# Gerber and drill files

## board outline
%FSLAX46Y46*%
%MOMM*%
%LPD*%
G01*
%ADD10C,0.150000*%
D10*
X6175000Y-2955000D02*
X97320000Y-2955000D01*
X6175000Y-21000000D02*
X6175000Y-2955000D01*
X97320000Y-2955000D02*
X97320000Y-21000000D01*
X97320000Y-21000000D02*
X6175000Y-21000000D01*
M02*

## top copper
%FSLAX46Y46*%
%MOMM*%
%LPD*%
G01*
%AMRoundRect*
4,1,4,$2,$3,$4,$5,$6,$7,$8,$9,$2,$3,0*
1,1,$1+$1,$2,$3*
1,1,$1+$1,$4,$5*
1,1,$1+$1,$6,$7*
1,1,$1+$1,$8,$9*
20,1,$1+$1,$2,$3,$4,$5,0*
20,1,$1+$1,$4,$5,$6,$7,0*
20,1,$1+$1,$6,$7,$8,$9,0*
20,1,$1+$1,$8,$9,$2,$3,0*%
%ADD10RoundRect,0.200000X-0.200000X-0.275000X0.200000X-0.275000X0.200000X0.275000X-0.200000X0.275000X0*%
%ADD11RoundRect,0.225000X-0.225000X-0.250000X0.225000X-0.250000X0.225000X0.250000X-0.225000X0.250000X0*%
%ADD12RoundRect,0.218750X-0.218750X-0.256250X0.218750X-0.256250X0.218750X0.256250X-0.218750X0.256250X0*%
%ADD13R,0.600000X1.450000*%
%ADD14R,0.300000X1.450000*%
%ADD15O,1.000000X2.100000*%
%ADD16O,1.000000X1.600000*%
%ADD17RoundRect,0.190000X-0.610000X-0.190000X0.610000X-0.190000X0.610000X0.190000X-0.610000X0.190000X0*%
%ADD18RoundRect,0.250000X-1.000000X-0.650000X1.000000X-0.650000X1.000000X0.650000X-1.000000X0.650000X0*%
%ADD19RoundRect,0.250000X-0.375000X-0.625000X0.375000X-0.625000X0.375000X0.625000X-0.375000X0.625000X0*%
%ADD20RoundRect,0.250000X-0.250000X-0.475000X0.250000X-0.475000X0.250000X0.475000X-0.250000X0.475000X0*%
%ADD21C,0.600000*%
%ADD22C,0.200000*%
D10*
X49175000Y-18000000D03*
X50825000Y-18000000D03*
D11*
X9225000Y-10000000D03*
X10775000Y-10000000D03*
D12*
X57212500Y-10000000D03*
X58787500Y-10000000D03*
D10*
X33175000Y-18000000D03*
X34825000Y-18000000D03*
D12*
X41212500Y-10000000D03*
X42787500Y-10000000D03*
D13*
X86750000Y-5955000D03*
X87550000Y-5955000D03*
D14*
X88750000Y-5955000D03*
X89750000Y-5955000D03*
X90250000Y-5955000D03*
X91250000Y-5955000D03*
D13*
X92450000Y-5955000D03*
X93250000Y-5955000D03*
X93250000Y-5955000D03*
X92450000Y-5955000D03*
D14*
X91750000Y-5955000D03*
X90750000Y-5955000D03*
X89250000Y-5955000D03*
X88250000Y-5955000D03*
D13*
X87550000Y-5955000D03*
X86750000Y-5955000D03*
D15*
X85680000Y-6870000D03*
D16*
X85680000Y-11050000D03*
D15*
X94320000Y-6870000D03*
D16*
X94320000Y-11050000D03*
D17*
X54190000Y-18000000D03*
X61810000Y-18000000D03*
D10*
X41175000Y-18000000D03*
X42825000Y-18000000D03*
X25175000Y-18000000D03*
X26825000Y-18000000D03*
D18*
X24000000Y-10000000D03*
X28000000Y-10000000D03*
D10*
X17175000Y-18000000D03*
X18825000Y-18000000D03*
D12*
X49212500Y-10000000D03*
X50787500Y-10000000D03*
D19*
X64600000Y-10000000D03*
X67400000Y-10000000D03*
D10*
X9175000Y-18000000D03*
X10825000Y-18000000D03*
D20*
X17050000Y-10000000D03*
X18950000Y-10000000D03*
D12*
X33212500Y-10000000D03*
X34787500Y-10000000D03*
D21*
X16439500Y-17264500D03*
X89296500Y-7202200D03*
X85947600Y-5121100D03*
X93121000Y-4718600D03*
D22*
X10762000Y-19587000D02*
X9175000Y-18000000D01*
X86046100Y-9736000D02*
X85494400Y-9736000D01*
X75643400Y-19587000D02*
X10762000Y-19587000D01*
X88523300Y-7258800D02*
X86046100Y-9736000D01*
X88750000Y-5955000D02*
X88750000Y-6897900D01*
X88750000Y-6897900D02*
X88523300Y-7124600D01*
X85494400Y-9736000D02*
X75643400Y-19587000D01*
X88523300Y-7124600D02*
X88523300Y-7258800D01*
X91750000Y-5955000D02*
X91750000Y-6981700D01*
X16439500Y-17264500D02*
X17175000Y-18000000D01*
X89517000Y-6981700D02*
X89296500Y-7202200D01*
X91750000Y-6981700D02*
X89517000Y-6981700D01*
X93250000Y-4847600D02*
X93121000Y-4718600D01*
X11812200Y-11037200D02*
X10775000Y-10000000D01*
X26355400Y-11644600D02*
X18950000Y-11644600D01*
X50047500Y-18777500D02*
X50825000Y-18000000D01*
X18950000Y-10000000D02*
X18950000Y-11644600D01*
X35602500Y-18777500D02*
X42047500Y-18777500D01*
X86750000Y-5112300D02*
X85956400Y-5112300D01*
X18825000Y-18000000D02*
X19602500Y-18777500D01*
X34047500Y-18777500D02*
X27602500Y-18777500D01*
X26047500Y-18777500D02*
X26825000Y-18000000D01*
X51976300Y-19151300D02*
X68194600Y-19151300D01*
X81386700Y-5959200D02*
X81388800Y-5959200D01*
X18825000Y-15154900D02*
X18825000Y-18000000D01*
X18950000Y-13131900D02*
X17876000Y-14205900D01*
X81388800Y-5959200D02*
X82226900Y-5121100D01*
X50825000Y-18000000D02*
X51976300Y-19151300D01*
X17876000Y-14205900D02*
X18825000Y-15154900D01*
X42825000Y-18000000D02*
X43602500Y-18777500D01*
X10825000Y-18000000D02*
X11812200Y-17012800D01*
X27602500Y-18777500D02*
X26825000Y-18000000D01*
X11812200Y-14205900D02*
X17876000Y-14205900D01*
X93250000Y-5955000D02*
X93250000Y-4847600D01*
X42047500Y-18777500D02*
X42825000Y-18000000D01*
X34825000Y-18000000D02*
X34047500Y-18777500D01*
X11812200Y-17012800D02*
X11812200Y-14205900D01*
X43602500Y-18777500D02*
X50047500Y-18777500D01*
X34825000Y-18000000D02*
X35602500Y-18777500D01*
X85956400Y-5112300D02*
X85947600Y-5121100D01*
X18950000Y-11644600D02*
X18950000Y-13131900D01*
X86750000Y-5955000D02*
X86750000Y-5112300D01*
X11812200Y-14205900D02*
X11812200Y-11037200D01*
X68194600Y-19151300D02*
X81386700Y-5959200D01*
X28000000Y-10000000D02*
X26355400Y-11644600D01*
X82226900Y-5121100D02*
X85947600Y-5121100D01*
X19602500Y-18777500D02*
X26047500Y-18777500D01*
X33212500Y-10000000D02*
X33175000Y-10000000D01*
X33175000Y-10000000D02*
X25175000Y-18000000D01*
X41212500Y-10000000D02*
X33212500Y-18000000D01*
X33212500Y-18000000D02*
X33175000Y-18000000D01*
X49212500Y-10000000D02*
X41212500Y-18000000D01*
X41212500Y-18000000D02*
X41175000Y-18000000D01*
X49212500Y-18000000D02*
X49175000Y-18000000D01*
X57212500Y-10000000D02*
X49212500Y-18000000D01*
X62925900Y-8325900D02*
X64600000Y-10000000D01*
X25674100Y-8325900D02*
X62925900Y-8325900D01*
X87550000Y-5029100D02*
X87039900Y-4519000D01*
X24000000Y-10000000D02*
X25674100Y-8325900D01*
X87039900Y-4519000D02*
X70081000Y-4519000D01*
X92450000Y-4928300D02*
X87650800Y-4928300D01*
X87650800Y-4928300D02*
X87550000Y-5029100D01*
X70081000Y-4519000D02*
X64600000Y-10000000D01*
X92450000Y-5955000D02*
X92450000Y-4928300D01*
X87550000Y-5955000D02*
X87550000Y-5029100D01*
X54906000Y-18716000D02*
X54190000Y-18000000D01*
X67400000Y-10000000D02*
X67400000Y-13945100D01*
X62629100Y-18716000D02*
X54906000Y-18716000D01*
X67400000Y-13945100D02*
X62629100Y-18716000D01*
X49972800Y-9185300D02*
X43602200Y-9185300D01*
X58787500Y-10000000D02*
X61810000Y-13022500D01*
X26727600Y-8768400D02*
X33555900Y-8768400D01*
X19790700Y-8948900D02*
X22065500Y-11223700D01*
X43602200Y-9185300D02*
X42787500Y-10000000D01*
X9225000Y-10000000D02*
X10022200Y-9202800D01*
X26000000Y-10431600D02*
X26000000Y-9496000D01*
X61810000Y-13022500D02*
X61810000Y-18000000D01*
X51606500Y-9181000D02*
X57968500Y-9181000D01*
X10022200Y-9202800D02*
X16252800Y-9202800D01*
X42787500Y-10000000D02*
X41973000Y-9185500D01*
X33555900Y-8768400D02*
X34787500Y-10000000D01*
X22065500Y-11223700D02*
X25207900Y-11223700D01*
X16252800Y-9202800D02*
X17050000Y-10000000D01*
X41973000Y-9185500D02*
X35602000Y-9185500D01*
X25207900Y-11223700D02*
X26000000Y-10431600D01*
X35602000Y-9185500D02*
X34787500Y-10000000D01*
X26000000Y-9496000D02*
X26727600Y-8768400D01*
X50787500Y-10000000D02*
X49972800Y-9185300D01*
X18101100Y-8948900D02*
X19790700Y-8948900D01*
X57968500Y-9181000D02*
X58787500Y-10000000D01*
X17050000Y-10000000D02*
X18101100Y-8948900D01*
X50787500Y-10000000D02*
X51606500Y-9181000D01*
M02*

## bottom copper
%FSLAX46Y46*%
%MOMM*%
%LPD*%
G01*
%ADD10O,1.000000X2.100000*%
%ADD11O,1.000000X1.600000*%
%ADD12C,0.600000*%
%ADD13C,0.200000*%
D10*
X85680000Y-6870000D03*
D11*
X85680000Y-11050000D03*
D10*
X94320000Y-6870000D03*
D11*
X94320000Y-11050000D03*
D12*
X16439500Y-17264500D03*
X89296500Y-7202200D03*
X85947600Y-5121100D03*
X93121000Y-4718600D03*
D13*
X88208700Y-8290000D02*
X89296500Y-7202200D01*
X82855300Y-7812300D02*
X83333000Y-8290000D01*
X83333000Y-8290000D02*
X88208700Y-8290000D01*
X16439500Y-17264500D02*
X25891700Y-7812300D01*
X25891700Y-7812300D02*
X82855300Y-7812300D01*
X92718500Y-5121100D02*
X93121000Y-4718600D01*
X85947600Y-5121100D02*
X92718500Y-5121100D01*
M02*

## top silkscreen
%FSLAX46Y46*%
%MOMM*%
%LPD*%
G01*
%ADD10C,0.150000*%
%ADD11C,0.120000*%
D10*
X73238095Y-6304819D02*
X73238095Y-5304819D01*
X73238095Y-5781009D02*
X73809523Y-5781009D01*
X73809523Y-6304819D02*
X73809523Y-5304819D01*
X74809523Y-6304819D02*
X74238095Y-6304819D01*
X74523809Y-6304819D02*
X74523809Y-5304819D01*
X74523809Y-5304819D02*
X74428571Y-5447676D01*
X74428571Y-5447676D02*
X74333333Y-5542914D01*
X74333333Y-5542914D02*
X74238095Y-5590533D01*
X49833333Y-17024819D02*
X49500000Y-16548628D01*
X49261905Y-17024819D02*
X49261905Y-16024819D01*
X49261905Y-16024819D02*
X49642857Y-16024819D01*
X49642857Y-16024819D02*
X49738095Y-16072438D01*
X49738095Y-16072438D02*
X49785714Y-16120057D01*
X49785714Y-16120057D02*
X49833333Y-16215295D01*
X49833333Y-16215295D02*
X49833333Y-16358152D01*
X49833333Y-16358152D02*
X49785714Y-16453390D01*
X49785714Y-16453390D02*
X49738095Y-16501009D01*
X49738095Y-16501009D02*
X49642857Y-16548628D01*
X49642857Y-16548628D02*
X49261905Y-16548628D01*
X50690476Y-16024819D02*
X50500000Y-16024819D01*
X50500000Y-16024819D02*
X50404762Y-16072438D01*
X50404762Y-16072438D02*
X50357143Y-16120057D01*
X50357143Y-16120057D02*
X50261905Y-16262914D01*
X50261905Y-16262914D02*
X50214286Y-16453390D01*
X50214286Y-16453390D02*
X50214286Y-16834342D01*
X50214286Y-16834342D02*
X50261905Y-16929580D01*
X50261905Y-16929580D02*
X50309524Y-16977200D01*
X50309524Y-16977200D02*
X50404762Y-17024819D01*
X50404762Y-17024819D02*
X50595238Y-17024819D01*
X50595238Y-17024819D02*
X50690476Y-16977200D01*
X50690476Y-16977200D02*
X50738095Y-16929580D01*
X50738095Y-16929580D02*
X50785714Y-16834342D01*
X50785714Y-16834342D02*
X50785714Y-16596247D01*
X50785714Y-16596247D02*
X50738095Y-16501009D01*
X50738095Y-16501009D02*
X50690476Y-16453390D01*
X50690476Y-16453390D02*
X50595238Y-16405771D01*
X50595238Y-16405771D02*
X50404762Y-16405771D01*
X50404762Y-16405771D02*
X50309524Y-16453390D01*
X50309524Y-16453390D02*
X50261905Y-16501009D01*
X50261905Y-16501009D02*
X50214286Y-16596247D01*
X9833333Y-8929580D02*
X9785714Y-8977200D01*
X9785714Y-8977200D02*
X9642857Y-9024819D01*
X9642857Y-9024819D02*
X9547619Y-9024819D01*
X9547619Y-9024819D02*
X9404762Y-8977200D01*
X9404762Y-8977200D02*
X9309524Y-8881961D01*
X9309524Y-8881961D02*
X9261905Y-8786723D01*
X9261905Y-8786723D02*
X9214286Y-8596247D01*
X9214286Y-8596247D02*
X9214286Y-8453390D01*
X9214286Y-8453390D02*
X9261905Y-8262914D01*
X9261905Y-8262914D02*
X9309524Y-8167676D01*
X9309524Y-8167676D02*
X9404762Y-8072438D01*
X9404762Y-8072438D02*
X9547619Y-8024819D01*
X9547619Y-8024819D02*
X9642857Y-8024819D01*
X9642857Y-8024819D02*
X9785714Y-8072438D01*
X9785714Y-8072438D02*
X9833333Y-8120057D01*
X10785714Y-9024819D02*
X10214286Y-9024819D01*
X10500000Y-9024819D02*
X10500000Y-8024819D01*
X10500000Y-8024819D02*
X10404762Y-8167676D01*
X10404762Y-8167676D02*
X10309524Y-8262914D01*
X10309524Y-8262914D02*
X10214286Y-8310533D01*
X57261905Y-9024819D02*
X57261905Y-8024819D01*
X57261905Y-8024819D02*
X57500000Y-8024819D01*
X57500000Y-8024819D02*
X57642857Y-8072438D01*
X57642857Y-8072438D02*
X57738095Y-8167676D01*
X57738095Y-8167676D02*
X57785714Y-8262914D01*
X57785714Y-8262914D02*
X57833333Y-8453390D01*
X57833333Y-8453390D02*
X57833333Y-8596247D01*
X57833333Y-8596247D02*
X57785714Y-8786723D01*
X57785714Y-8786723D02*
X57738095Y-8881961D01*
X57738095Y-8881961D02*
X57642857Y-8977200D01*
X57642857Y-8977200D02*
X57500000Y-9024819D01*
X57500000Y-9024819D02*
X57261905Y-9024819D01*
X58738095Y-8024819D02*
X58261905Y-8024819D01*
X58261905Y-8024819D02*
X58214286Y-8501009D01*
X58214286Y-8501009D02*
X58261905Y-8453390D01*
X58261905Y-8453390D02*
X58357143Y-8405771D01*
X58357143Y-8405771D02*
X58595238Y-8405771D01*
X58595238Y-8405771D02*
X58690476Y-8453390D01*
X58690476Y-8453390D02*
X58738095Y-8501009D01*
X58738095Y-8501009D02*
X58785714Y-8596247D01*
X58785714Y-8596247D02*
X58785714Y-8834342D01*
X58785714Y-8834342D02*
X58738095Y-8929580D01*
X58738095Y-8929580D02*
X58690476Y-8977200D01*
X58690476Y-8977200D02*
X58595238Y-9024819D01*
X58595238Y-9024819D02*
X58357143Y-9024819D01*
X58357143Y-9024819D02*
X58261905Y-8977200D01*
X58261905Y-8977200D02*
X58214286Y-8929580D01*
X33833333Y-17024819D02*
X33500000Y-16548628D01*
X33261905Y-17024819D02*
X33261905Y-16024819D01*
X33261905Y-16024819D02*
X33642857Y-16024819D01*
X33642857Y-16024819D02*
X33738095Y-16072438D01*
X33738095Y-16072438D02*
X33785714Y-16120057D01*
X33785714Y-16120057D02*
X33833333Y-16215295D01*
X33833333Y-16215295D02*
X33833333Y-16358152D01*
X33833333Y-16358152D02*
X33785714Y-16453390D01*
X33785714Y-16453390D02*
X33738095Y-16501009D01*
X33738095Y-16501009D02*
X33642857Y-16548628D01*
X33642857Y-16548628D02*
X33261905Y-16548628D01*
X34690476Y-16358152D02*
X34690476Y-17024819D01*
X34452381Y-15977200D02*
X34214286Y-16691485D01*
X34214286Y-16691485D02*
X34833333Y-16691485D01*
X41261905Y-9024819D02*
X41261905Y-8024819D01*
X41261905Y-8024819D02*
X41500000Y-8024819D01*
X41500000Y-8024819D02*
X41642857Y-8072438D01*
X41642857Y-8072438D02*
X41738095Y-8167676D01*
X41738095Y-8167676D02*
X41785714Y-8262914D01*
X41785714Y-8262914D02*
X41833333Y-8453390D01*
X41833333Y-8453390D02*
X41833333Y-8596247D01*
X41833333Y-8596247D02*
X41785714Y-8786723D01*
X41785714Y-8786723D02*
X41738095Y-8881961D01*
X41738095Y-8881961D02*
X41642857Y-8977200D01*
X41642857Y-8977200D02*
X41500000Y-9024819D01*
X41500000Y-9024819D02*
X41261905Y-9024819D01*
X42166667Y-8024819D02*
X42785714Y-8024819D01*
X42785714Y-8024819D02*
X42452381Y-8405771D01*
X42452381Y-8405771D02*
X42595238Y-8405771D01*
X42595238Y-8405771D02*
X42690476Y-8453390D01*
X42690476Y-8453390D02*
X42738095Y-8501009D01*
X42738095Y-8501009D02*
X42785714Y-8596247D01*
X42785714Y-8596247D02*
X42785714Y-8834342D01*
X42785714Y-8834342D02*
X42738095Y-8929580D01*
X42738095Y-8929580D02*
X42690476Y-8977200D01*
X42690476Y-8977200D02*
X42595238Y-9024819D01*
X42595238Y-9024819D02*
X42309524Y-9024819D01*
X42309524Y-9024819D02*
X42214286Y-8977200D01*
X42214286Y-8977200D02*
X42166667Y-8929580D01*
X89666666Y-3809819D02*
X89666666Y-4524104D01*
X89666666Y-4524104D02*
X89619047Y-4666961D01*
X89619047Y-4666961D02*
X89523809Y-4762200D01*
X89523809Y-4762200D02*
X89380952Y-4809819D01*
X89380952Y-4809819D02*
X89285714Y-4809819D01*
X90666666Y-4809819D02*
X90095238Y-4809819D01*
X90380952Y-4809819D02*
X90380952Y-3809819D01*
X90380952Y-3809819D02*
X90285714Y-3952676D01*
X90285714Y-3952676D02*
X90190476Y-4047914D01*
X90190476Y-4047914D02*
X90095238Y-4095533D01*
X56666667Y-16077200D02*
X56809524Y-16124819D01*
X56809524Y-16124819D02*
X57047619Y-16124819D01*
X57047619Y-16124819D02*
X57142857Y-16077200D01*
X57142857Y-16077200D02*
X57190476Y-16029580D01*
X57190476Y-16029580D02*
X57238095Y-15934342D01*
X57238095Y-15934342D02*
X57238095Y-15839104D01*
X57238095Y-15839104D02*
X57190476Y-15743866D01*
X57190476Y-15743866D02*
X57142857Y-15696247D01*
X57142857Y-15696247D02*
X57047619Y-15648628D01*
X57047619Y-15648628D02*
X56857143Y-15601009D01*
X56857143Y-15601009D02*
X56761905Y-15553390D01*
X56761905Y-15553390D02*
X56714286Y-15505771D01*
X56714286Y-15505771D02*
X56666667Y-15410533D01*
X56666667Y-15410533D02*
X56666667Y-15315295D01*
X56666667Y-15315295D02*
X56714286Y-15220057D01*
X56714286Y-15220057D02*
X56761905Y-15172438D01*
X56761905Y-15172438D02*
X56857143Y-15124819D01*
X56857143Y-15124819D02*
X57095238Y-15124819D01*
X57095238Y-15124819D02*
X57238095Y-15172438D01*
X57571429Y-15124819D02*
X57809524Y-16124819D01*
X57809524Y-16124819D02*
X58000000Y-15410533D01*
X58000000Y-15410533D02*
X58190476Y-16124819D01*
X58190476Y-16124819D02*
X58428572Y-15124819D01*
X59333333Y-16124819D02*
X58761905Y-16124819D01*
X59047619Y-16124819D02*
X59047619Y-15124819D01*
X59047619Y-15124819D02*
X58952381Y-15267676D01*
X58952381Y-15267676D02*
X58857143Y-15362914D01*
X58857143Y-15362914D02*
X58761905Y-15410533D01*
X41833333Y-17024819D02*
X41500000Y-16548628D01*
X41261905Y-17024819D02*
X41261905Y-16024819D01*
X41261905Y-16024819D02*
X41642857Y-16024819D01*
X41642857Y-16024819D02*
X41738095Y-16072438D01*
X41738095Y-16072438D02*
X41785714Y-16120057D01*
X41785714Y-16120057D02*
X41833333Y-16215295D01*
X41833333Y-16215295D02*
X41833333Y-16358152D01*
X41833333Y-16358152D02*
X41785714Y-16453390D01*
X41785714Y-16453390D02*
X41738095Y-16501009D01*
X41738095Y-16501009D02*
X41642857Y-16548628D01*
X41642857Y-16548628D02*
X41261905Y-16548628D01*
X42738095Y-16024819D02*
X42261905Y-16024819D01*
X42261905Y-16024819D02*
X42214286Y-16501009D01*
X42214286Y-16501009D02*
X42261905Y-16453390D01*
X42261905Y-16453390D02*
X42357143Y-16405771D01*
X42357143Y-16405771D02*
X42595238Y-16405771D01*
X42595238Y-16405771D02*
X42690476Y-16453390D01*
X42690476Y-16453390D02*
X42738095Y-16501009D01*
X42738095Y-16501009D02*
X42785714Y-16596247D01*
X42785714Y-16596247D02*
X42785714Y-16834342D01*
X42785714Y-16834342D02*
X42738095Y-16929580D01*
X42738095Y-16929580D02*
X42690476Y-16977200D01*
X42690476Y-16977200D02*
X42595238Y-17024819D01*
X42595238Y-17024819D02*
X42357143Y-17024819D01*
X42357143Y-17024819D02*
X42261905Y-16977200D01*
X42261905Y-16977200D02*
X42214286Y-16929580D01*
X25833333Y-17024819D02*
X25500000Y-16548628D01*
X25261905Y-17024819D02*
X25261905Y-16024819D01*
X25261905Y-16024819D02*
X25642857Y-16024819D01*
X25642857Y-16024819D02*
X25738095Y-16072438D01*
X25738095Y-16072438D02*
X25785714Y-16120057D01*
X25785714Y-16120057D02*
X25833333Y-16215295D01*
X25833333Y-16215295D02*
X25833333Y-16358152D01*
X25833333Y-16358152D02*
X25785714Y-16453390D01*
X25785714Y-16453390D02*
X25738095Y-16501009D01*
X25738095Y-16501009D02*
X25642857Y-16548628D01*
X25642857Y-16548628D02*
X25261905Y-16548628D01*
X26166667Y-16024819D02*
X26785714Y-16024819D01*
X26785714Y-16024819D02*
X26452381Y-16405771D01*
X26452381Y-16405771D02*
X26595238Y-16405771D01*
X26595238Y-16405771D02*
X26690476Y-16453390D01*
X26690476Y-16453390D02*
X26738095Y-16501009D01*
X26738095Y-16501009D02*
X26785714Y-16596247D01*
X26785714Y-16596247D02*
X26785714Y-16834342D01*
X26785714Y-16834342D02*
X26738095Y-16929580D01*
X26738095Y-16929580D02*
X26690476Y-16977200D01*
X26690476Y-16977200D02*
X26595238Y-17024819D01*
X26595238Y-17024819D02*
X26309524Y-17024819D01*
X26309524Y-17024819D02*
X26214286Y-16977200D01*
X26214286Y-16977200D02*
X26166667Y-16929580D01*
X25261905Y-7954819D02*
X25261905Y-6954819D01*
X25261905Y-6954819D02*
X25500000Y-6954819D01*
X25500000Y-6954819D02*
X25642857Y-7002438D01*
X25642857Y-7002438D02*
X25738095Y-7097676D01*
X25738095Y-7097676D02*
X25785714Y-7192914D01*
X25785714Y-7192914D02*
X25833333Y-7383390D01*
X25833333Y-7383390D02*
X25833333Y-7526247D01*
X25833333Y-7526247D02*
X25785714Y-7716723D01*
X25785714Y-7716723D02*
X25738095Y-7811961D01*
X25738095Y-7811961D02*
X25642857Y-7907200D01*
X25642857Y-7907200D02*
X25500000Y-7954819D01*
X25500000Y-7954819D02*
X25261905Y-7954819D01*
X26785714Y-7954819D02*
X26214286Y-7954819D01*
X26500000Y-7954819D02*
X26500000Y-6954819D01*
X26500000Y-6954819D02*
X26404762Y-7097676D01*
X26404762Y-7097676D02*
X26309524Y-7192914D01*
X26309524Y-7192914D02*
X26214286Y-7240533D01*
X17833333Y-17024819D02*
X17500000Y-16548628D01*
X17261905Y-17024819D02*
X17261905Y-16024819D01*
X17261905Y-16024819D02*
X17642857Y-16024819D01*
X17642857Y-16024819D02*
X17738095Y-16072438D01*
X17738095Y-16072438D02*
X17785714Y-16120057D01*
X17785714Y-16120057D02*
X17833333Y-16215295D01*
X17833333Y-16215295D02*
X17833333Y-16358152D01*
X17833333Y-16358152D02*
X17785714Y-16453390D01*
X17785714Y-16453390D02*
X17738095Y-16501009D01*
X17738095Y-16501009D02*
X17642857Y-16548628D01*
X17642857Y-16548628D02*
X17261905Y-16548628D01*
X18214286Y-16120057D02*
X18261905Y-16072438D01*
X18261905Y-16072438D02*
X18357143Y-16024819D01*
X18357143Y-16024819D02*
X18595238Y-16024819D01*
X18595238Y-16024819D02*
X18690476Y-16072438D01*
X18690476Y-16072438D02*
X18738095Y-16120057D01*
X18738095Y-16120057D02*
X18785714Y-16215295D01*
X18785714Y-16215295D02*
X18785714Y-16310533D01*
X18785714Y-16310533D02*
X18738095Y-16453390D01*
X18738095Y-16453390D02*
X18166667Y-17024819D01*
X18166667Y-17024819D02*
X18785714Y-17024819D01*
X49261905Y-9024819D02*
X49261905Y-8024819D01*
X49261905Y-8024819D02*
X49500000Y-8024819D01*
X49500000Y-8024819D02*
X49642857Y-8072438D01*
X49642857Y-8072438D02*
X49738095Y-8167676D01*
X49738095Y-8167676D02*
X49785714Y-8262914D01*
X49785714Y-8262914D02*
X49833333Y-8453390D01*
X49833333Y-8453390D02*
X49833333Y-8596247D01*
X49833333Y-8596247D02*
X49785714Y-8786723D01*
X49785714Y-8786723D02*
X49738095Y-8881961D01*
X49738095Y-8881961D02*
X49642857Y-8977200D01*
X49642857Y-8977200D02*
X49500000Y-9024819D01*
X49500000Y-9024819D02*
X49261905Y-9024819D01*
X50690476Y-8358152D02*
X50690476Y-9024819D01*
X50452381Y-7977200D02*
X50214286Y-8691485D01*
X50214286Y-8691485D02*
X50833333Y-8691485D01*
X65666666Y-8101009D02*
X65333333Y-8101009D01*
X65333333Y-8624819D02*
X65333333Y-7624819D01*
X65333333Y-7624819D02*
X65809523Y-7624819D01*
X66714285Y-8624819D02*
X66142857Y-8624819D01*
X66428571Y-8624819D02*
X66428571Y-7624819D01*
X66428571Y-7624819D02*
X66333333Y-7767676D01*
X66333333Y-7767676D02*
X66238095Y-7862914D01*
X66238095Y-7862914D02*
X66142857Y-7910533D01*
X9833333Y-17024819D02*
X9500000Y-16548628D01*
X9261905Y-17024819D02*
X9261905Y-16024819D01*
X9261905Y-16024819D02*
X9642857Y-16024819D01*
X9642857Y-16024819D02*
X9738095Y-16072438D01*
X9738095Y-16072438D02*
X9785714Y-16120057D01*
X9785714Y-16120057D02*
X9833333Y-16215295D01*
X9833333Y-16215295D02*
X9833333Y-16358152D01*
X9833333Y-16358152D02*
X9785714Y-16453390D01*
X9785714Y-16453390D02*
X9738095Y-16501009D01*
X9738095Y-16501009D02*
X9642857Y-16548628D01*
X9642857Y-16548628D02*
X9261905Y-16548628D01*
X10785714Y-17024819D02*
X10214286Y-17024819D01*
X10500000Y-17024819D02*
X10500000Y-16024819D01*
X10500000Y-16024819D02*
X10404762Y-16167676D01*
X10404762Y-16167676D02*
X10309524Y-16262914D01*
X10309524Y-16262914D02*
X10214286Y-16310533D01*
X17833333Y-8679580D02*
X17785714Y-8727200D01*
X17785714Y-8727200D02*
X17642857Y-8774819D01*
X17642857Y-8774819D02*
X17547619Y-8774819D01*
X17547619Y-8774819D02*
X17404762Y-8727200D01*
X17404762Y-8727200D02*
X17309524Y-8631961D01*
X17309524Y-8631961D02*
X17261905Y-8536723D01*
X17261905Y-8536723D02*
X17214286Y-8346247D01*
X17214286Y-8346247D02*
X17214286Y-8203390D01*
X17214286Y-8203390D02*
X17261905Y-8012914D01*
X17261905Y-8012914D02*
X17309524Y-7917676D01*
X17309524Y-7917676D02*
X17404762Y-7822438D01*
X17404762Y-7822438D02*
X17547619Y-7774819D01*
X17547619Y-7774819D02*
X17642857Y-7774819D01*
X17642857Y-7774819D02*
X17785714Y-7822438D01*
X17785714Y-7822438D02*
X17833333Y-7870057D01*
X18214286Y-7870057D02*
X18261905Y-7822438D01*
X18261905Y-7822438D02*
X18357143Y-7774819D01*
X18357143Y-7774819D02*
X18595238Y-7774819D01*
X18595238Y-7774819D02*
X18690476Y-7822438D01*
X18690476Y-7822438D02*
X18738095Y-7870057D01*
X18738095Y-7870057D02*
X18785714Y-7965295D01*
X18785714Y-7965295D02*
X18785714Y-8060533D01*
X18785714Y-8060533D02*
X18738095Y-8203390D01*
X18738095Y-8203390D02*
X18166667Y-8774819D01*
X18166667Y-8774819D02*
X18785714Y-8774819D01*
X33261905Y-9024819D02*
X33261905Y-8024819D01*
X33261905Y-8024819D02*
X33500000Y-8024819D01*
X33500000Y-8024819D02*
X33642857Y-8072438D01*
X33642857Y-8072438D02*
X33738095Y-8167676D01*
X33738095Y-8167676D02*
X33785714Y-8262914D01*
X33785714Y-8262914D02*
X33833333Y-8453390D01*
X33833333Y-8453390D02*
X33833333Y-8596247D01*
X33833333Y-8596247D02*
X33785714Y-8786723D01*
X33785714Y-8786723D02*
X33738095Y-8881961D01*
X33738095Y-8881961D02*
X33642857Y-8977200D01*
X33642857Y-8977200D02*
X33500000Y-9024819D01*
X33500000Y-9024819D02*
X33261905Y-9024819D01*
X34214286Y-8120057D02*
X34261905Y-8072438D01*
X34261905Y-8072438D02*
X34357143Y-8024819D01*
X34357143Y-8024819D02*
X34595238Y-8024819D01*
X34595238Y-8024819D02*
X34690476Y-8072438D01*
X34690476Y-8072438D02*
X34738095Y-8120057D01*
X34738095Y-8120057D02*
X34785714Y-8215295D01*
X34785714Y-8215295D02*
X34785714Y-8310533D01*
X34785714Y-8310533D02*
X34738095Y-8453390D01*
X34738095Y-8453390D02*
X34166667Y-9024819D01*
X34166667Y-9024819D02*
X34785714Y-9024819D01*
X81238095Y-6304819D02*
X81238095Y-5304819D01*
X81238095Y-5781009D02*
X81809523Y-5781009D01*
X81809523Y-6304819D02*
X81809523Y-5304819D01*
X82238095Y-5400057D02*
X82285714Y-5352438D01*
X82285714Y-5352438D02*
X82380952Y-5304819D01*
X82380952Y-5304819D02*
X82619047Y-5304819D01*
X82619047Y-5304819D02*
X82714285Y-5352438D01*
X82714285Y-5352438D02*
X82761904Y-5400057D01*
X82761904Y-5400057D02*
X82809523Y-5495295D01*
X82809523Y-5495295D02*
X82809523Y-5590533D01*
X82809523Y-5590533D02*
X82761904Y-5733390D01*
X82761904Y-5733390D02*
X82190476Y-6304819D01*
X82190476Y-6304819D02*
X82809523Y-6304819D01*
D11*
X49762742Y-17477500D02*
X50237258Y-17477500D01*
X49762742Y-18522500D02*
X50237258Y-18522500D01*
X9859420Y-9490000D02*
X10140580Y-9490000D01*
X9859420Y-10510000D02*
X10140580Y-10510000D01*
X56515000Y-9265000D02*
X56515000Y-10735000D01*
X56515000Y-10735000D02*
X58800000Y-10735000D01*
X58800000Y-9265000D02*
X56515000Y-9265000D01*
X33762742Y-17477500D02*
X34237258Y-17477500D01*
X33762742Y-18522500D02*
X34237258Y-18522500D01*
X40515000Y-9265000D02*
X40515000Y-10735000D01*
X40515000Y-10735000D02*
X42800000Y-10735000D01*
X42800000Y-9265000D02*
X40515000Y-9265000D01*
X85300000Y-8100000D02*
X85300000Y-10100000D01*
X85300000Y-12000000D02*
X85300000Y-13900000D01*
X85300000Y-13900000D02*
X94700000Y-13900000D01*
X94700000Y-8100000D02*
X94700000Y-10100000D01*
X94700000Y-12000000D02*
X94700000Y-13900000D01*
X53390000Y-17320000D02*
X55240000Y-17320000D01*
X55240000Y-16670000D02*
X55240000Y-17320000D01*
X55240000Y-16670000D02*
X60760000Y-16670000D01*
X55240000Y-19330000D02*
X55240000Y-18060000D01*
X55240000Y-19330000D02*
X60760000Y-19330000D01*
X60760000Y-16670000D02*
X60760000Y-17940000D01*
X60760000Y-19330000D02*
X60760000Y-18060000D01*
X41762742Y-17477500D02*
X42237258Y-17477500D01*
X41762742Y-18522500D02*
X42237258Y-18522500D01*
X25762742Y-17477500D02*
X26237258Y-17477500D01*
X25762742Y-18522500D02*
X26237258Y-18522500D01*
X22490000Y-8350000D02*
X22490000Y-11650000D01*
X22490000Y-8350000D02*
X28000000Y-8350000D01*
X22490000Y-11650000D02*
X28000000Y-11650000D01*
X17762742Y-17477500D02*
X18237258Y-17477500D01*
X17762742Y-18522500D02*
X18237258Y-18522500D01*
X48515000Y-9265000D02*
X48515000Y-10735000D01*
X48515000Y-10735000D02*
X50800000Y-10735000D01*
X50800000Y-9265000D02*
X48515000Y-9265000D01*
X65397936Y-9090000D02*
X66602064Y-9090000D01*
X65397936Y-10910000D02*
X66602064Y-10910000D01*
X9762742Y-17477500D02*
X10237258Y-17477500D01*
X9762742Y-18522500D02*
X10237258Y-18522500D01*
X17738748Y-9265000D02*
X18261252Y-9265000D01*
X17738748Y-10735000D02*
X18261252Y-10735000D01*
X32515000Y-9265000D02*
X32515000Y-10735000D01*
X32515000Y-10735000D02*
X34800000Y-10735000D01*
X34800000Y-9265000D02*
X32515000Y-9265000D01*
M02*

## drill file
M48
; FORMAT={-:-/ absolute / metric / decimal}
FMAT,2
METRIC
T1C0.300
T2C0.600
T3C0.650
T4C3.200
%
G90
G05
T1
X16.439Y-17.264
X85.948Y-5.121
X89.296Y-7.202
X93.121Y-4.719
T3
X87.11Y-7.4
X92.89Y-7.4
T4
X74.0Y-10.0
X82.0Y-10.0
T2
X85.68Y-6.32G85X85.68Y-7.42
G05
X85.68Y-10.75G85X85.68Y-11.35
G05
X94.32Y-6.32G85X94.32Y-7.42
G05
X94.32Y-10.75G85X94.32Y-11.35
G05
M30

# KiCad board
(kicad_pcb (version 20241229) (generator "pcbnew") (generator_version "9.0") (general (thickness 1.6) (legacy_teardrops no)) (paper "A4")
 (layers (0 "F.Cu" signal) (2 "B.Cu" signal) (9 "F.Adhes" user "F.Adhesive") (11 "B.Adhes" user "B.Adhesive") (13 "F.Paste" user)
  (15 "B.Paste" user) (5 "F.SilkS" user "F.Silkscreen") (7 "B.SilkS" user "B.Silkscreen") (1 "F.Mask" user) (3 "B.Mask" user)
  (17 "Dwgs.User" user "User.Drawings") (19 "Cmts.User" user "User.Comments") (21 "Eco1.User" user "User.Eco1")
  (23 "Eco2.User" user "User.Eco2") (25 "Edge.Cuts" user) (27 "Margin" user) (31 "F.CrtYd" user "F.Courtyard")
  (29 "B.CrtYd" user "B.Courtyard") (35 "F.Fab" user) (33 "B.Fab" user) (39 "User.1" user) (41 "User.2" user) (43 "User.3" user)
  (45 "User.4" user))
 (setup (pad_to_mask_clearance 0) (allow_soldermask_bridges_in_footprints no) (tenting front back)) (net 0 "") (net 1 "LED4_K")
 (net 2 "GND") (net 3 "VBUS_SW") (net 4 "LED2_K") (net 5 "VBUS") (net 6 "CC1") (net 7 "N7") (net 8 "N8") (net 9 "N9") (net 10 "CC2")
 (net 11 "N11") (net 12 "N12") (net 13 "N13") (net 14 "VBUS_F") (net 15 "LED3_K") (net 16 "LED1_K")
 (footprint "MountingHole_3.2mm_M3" (layer "F.Cu") (at 74 10)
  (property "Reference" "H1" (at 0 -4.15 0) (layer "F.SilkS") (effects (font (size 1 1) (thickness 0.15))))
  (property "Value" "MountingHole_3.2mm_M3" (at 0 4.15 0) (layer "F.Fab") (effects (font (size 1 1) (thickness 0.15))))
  (pad "" np_thru_hole circle (at 0 0) (size 3.2 3.2) (drill 3.2) (layers "*.Cu" "*.Mask")))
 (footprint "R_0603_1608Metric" (layer "F.Cu") (at 50 18)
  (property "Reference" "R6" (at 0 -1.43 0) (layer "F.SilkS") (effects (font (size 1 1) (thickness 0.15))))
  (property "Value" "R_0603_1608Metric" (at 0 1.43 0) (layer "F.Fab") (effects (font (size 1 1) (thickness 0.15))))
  (fp_line (start -0.237258 -0.5225) (end 0.237258 -0.5225) (stroke (width 0.12) (type solid)) (layer "F.SilkS"))
  (fp_line (start -0.237258 0.5225) (end 0.237258 0.5225) (stroke (width 0.12) (type solid)) (layer "F.SilkS"))
  (pad "1" smd roundrect (at -0.825 0) (size 0.8 0.95) (layers "F.Cu" "F.Mask" "F.Paste") (roundrect_rratio 0.25) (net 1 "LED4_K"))
  (pad "2" smd roundrect (at 0.825 0) (size 0.8 0.95) (layers "F.Cu" "F.Mask" "F.Paste") (roundrect_rratio 0.25) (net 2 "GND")))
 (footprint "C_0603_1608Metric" (layer "F.Cu") (at 10 10)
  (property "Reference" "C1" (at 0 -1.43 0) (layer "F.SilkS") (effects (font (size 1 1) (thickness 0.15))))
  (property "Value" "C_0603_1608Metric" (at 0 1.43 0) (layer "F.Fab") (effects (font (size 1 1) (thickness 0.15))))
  (fp_line (start -0.14058 -0.51) (end 0.14058 -0.51) (stroke (width 0.12) (type solid)) (layer "F.SilkS"))
  (fp_line (start -0.14058 0.51) (end 0.14058 0.51) (stroke (width 0.12) (type solid)) (layer "F.SilkS"))
  (pad "1" smd roundrect (at -0.775 0) (size 0.9 0.95) (layers "F.Cu" "F.Mask" "F.Paste") (roundrect_rratio 0.25) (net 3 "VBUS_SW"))
  (pad "2" smd roundrect (at 0.775 0) (size 0.9 0.95) (layers "F.Cu" "F.Mask" "F.Paste") (roundrect_rratio 0.25) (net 2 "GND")))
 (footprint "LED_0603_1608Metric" (layer "F.Cu") (at 58 10)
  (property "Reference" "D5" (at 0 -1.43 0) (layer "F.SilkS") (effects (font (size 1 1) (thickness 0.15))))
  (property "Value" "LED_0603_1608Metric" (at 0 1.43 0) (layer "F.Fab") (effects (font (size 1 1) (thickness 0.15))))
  (fp_line (start -1.485 -0.735) (end -1.485 0.735) (stroke (width 0.12) (type solid)) (layer "F.SilkS"))
  (fp_line (start -1.485 0.735) (end 0.8 0.735) (stroke (width 0.12) (type solid)) (layer "F.SilkS"))
  (fp_line (start 0.8 -0.735) (end -1.485 -0.735) (stroke (width 0.12) (type solid)) (layer "F.SilkS"))
  (pad "1" smd roundrect (at -0.7875 0) (size 0.875 0.95) (layers "F.Cu" "F.Mask" "F.Paste") (roundrect_rratio 0.25) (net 1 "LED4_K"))
  (pad "2" smd roundrect (at 0.7875 0) (size 0.875 0.95) (layers "F.Cu" "F.Mask" "F.Paste") (roundrect_rratio 0.25) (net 3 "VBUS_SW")))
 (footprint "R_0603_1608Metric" (layer "F.Cu") (at 34 18)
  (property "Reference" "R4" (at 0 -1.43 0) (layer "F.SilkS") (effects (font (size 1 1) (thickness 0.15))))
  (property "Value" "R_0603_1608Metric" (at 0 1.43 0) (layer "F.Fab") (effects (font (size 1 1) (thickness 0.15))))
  (fp_line (start -0.237258 -0.5225) (end 0.237258 -0.5225) (stroke (width 0.12) (type solid)) (layer "F.SilkS"))
  (fp_line (start -0.237258 0.5225) (end 0.237258 0.5225) (stroke (width 0.12) (type solid)) (layer "F.SilkS"))
  (pad "1" smd roundrect (at -0.825 0) (size 0.8 0.95) (layers "F.Cu" "F.Mask" "F.Paste") (roundrect_rratio 0.25) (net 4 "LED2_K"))
  (pad "2" smd roundrect (at 0.825 0) (size 0.8 0.95) (layers "F.Cu" "F.Mask" "F.Paste") (roundrect_rratio 0.25) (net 2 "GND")))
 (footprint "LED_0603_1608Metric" (layer "F.Cu") (at 42 10)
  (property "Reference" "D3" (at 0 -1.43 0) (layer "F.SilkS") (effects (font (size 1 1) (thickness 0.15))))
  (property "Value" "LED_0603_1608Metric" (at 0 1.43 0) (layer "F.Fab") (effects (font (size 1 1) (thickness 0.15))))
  (fp_line (start -1.485 -0.735) (end -1.485 0.735) (stroke (width 0.12) (type solid)) (layer "F.SilkS"))
  (fp_line (start -1.485 0.735) (end 0.8 0.735) (stroke (width 0.12) (type solid)) (layer "F.SilkS"))
  (fp_line (start 0.8 -0.735) (end -1.485 -0.735) (stroke (width 0.12) (type solid)) (layer "F.SilkS"))
  (pad "1" smd roundrect (at -0.7875 0) (size 0.875 0.95) (layers "F.Cu" "F.Mask" "F.Paste") (roundrect_rratio 0.25) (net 4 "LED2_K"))
  (pad "2" smd roundrect (at 0.7875 0) (size 0.875 0.95) (layers "F.Cu" "F.Mask" "F.Paste") (roundrect_rratio 0.25) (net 3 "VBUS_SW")))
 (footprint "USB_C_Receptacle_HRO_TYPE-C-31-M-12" (layer "F.Cu") (at 90 10)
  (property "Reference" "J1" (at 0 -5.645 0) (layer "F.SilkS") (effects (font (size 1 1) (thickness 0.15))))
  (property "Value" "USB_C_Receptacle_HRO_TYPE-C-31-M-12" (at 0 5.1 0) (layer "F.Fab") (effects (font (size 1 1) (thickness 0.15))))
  (fp_line (start -4.7 -1.9) (end -4.7 0.1) (stroke (width 0.12) (type solid)) (layer "F.SilkS"))
  (fp_line (start -4.7 2) (end -4.7 3.9) (stroke (width 0.12) (type solid)) (layer "F.SilkS"))
  (fp_line (start -4.7 3.9) (end 4.7 3.9) (stroke (width 0.12) (type solid)) (layer "F.SilkS"))
  (fp_line (start 4.7 -1.9) (end 4.7 0.1) (stroke (width 0.12) (type solid)) (layer "F.SilkS"))
  (fp_line (start 4.7 2) (end 4.7 3.9) (stroke (width 0.12) (type solid)) (layer "F.SilkS"))
  (pad "" np_thru_hole circle (at -2.89 -2.6) (size 0.65 0.65) (drill 0.65) (layers "*.Cu" "*.Mask"))
  (pad "" np_thru_hole circle (at 2.89 -2.6) (size 0.65 0.65) (drill 0.65) (layers "*.Cu" "*.Mask"))
  (pad "A1" smd rect (at -3.25 -4.045) (size 0.6 1.45) (layers "F.Cu" "F.Mask" "F.Paste") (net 2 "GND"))
  (pad "A4" smd rect (at -2.45 -4.045) (size 0.6 1.45) (layers "F.Cu" "F.Mask" "F.Paste") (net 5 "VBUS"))
  (pad "A5" smd rect (at -1.25 -4.045) (size 0.3 1.45) (layers "F.Cu" "F.Mask" "F.Paste") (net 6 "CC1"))
  (pad "A6" smd rect (at -0.25 -4.045) (size 0.3 1.45) (layers "F.Cu" "F.Mask" "F.Paste") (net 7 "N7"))
  (pad "A7" smd rect (at 0.25 -4.045) (size 0.3 1.45) (layers "F.Cu" "F.Mask" "F.Paste") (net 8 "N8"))
  (pad "A8" smd rect (at 1.25 -4.045) (size 0.3 1.45) (layers "F.Cu" "F.Mask" "F.Paste") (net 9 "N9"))
  (pad "A9" smd rect (at 2.45 -4.045) (size 0.6 1.45) (layers "F.Cu" "F.Mask" "F.Paste") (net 5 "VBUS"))
  (pad "A12" smd rect (at 3.25 -4.045) (size 0.6 1.45) (layers "F.Cu" "F.Mask" "F.Paste") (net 2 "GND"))
  (pad "B1" smd rect (at 3.25 -4.045) (size 0.6 1.45) (layers "F.Cu" "F.Mask" "F.Paste") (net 2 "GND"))
  (pad "B4" smd rect (at 2.45 -4.045) (size 0.6 1.45) (layers "F.Cu" "F.Mask" "F.Paste") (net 5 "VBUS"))
  (pad "B5" smd rect (at 1.75 -4.045) (size 0.3 1.45) (layers "F.Cu" "F.Mask" "F.Paste") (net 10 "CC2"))
  (pad "B6" smd rect (at 0.75 -4.045) (size 0.3 1.45) (layers "F.Cu" "F.Mask" "F.Paste") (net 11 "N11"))
  (pad "B7" smd rect (at -0.75 -4.045) (size 0.3 1.45) (layers "F.Cu" "F.Mask" "F.Paste") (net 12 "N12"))
  (pad "B8" smd rect (at -1.75 -4.045) (size 0.3 1.45) (layers "F.Cu" "F.Mask" "F.Paste") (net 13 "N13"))
  (pad "B9" smd rect (at -2.45 -4.045) (size 0.6 1.45) (layers "F.Cu" "F.Mask" "F.Paste") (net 5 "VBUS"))
  (pad "B12" smd rect (at -3.25 -4.045) (size 0.6 1.45) (layers "F.Cu" "F.Mask" "F.Paste") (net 2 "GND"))
  (pad "S1" thru_hole oval (at -4.32 -3.13) (size 1 2.1) (drill oval 0.6 1.7) (layers "*.Cu" "*.Mask") (remove_unused_layers no))
  (pad "S1" thru_hole oval (at -4.32 1.05) (size 1 1.6) (drill oval 0.6 1.2) (layers "*.Cu" "*.Mask") (remove_unused_layers no))
  (pad "S1" thru_hole oval (at 4.32 -3.13) (size 1 2.1) (drill oval 0.6 1.7) (layers "*.Cu" "*.Mask") (remove_unused_layers no))
  (pad "S1" thru_hole oval (at 4.32 1.05) (size 1 1.6) (drill oval 0.6 1.2) (layers "*.Cu" "*.Mask") (remove_unused_layers no)))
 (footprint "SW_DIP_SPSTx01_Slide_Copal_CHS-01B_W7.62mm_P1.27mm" (layer "F.Cu") (at 58 18)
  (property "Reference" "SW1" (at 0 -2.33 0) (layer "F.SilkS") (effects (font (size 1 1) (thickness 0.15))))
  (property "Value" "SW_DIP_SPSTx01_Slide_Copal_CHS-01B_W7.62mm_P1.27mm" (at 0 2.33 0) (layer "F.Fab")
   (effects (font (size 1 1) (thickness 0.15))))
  (fp_line (start -4.61 -0.68) (end -2.76 -0.68) (stroke (width 0.12) (type solid)) (layer "F.SilkS"))
  (fp_line (start -2.76 -1.33) (end -2.76 -0.68) (stroke (width 0.12) (type solid)) (layer "F.SilkS"))
  (fp_line (start -2.76 -1.33) (end 2.76 -1.33) (stroke (width 0.12) (type solid)) (layer "F.SilkS"))
  (fp_line (start -2.76 1.33) (end -2.76 0.06) (stroke (width 0.12) (type solid)) (layer "F.SilkS"))
  (fp_line (start -2.76 1.33) (end 2.76 1.33) (stroke (width 0.12) (type solid)) (layer "F.SilkS"))
  (fp_line (start 2.76 -1.33) (end 2.76 -0.06) (stroke (width 0.12) (type solid)) (layer "F.SilkS"))
  (fp_line (start 2.76 1.33) (end 2.76 0.06) (stroke (width 0.12) (type solid)) (layer "F.SilkS"))
  (pad "1" smd roundrect (at -3.81 0) (size 1.6 0.76) (layers "F.Cu" "F.Mask" "F.Paste") (roundrect_rratio 0.25) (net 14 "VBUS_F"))
  (pad "2" smd roundrect (at 3.81 0) (size 1.6 0.76) (layers "F.Cu" "F.Mask" "F.Paste") (roundrect_rratio 0.25) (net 3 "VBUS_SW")))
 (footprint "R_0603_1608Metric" (layer "F.Cu") (at 42 18)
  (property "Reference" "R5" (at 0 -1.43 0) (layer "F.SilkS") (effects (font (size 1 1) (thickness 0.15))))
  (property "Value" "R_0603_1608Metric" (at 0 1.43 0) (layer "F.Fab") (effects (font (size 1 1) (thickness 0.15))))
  (fp_line (start -0.237258 -0.5225) (end 0.237258 -0.5225) (stroke (width 0.12) (type solid)) (layer "F.SilkS"))
  (fp_line (start -0.237258 0.5225) (end 0.237258 0.5225) (stroke (width 0.12) (type solid)) (layer "F.SilkS"))
  (pad "1" smd roundrect (at -0.825 0) (size 0.8 0.95) (layers "F.Cu" "F.Mask" "F.Paste") (roundrect_rratio 0.25) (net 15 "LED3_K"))
  (pad "2" smd roundrect (at 0.825 0) (size 0.8 0.95) (layers "F.Cu" "F.Mask" "F.Paste") (roundrect_rratio 0.25) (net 2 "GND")))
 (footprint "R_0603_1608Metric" (layer "F.Cu") (at 26 18)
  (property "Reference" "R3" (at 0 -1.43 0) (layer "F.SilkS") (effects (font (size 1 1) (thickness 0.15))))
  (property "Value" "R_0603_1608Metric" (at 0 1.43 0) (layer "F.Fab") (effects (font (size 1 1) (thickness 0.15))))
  (fp_line (start -0.237258 -0.5225) (end 0.237258 -0.5225) (stroke (width 0.12) (type solid)) (layer "F.SilkS"))
  (fp_line (start -0.237258 0.5225) (end 0.237258 0.5225) (stroke (width 0.12) (type solid)) (layer "F.SilkS"))
  (pad "1" smd roundrect (at -0.825 0) (size 0.8 0.95) (layers "F.Cu" "F.Mask" "F.Paste") (roundrect_rratio 0.25) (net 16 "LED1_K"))
  (pad "2" smd roundrect (at 0.825 0) (size 0.8 0.95) (layers "F.Cu" "F.Mask" "F.Paste") (roundrect_rratio 0.25) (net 2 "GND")))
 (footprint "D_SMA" (layer "F.Cu") (at 26 10)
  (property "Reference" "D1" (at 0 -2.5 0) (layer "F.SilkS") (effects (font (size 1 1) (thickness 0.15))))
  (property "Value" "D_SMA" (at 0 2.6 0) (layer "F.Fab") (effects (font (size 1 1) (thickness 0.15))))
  (fp_line (start -3.51 -1.65) (end -3.51 1.65) (stroke (width 0.12) (type solid)) (layer "F.SilkS"))
  (fp_line (start -3.51 -1.65) (end 2 -1.65) (stroke (width 0.12) (type solid)) (layer "F.SilkS"))
  (fp_line (start -3.51 1.65) (end 2 1.65) (stroke (width 0.12) (type solid)) (layer "F.SilkS"))
  (pad "1" smd roundrect (at -2 0) (size 2.5 1.8) (layers "F.Cu" "F.Mask" "F.Paste") (roundrect_rratio 0.1388888889) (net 5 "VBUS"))
  (pad "2" smd roundrect (at 2 0) (size 2.5 1.8) (layers "F.Cu" "F.Mask" "F.Paste") (roundrect_rratio 0.1388888889) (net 2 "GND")))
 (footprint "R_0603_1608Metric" (layer "F.Cu") (at 18 18)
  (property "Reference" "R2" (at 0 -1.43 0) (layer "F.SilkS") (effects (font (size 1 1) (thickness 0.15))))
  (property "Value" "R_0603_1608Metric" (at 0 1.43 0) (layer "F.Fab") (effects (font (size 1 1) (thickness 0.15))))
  (fp_line (start -0.237258 -0.5225) (end 0.237258 -0.5225) (stroke (width 0.12) (type solid)) (layer "F.SilkS"))
  (fp_line (start -0.237258 0.5225) (end 0.237258 0.5225) (stroke (width 0.12) (type solid)) (layer "F.SilkS"))
  (pad "1" smd roundrect (at -0.825 0) (size 0.8 0.95) (layers "F.Cu" "F.Mask" "F.Paste") (roundrect_rratio 0.25) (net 10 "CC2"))
  (pad "2" smd roundrect (at 0.825 0) (size 0.8 0.95) (layers "F.Cu" "F.Mask" "F.Paste") (roundrect_rratio 0.25) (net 2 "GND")))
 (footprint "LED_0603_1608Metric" (layer "F.Cu") (at 50 10)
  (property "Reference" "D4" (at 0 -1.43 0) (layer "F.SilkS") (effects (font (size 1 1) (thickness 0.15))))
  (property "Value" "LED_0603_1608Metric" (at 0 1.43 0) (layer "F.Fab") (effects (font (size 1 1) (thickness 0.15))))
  (fp_line (start -1.485 -0.735) (end -1.485 0.735) (stroke (width 0.12) (type solid)) (layer "F.SilkS"))
  (fp_line (start -1.485 0.735) (end 0.8 0.735) (stroke (width 0.12) (type solid)) (layer "F.SilkS"))
  (fp_line (start 0.8 -0.735) (end -1.485 -0.735) (stroke (width 0.12) (type solid)) (layer "F.SilkS"))
  (pad "1" smd roundrect (at -0.7875 0) (size 0.875 0.95) (layers "F.Cu" "F.Mask" "F.Paste") (roundrect_rratio 0.25) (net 15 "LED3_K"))
  (pad "2" smd roundrect (at 0.7875 0) (size 0.875 0.95) (layers "F.Cu" "F.Mask" "F.Paste") (roundrect_rratio 0.25) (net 3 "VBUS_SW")))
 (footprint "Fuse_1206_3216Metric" (layer "F.Cu") (at 66 10)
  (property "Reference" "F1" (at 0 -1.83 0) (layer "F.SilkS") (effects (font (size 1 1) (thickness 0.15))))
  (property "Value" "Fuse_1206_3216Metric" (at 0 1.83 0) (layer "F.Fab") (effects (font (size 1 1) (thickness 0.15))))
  (fp_line (start -0.602064 -0.91) (end 0.602064 -0.91) (stroke (width 0.12) (type solid)) (layer "F.SilkS"))
  (fp_line (start -0.602064 0.91) (end 0.602064 0.91) (stroke (width 0.12) (type solid)) (layer "F.SilkS"))
  (pad "1" smd roundrect (at -1.4 0) (size 1.25 1.75) (layers "F.Cu" "F.Mask" "F.Paste") (roundrect_rratio 0.2) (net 5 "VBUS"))
  (pad "2" smd roundrect (at 1.4 0) (size 1.25 1.75) (layers "F.Cu" "F.Mask" "F.Paste") (roundrect_rratio 0.2) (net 14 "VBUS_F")))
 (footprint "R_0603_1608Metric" (layer "F.Cu") (at 10 18)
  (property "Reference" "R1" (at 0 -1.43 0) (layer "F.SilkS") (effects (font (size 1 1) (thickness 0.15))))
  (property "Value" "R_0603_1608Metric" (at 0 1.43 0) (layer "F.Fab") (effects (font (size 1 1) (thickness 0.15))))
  (fp_line (start -0.237258 -0.5225) (end 0.237258 -0.5225) (stroke (width 0.12) (type solid)) (layer "F.SilkS"))
  (fp_line (start -0.237258 0.5225) (end 0.237258 0.5225) (stroke (width 0.12) (type solid)) (layer "F.SilkS"))
  (pad "1" smd roundrect (at -0.825 0) (size 0.8 0.95) (layers "F.Cu" "F.Mask" "F.Paste") (roundrect_rratio 0.25) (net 6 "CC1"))
  (pad "2" smd roundrect (at 0.825 0) (size 0.8 0.95) (layers "F.Cu" "F.Mask" "F.Paste") (roundrect_rratio 0.25) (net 2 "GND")))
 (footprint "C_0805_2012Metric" (layer "F.Cu") (at 18 10)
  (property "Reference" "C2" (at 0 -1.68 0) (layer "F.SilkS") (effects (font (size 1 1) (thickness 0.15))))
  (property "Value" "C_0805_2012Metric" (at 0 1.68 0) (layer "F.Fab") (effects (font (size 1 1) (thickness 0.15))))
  (fp_line (start -0.261252 -0.735) (end 0.261252 -0.735) (stroke (width 0.12) (type solid)) (layer "F.SilkS"))
  (fp_line (start -0.261252 0.735) (end 0.261252 0.735) (stroke (width 0.12) (type solid)) (layer "F.SilkS"))
  (pad "1" smd roundrect (at -0.95 0) (size 1 1.45) (layers "F.Cu" "F.Mask" "F.Paste") (roundrect_rratio 0.25) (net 3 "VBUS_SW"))
  (pad "2" smd roundrect (at 0.95 0) (size 1 1.45) (layers "F.Cu" "F.Mask" "F.Paste") (roundrect_rratio 0.25) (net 2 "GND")))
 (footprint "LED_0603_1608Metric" (layer "F.Cu") (at 34 10)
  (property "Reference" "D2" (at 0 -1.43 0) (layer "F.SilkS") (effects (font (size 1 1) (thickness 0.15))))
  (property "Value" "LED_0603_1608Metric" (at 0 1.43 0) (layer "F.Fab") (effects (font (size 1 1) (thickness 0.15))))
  (fp_line (start -1.485 -0.735) (end -1.485 0.735) (stroke (width 0.12) (type solid)) (layer "F.SilkS"))
  (fp_line (start -1.485 0.735) (end 0.8 0.735) (stroke (width 0.12) (type solid)) (layer "F.SilkS"))
  (fp_line (start 0.8 -0.735) (end -1.485 -0.735) (stroke (width 0.12) (type solid)) (layer "F.SilkS"))
  (pad "1" smd roundrect (at -0.7875 0) (size 0.875 0.95) (layers "F.Cu" "F.Mask" "F.Paste") (roundrect_rratio 0.25) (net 16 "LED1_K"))
  (pad "2" smd roundrect (at 0.7875 0) (size 0.875 0.95) (layers "F.Cu" "F.Mask" "F.Paste") (roundrect_rratio 0.25) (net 3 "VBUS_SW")))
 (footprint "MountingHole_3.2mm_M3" (layer "F.Cu") (at 82 10)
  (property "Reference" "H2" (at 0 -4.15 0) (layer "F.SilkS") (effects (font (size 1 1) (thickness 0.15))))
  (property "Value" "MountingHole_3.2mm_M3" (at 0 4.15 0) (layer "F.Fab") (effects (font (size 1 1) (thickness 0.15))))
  (pad "" np_thru_hole circle (at 0 0) (size 3.2 3.2) (drill 3.2) (layers "*.Cu" "*.Mask")))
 (gr_line (start 6.175 2.955) (end 97.32 2.955) (stroke (width 0.15) (type default)) (layer "Edge.Cuts"))
 (gr_line (start 6.175 21) (end 6.175 2.955) (stroke (width 0.15) (type default)) (layer "Edge.Cuts"))
 (gr_line (start 97.32 2.955) (end 97.32 21) (stroke (width 0.15) (type default)) (layer "Edge.Cuts"))
 (gr_line (start 97.32 21) (end 6.175 21) (stroke (width 0.15) (type default)) (layer "Edge.Cuts"))
 (segment (start 10.762 19.587) (end 9.175 18) (width 0.2) (layer "F.Cu") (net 6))
 (segment (start 86.0461 9.736) (end 85.4944 9.736) (width 0.2) (layer "F.Cu") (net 6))
 (segment (start 75.6434 19.587) (end 10.762 19.587) (width 0.2) (layer "F.Cu") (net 6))
 (segment (start 88.5233 7.2588) (end 86.0461 9.736) (width 0.2) (layer "F.Cu") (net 6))
 (segment (start 88.75 5.955) (end 88.75 6.8979) (width 0.2) (layer "F.Cu") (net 6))
 (segment (start 88.75 6.8979) (end 88.5233 7.1246) (width 0.2) (layer "F.Cu") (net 6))
 (segment (start 85.4944 9.736) (end 75.6434 19.587) (width 0.2) (layer "F.Cu") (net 6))
 (segment (start 88.5233 7.1246) (end 88.5233 7.2588) (width 0.2) (layer "F.Cu") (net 6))
 (segment (start 91.75 5.955) (end 91.75 6.9817) (width 0.2) (layer "F.Cu") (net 10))
 (segment (start 16.4395 17.2645) (end 17.175 18) (width 0.2) (layer "F.Cu") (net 10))
 (segment (start 89.517 6.9817) (end 89.2965 7.2022) (width 0.2) (layer "F.Cu") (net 10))
 (segment (start 91.75 6.9817) (end 89.517 6.9817) (width 0.2) (layer "F.Cu") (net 10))
 (via (at 16.4395 17.2645) (size 0.6) (drill 0.3) (layers "F.Cu" "B.Cu") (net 10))
 (via (at 89.2965 7.2022) (size 0.6) (drill 0.3) (layers "F.Cu" "B.Cu") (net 10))
 (segment (start 88.2087 8.29) (end 89.2965 7.2022) (width 0.2) (layer "B.Cu") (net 10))
 (segment (start 82.8553 7.8123) (end 83.333 8.29) (width 0.2) (layer "B.Cu") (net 10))
 (segment (start 83.333 8.29) (end 88.2087 8.29) (width 0.2) (layer "B.Cu") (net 10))
 (segment (start 16.4395 17.2645) (end 25.8917 7.8123) (width 0.2) (layer "B.Cu") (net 10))
 (segment (start 25.8917 7.8123) (end 82.8553 7.8123) (width 0.2) (layer "B.Cu") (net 10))
 (segment (start 93.25 4.8476) (end 93.121 4.7186) (width 0.2) (layer "F.Cu") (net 2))
 (segment (start 11.8122 11.0372) (end 10.775 10) (width 0.2) (layer "F.Cu") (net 2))
 (segment (start 26.3554 11.6446) (end 18.95 11.6446) (width 0.2) (layer "F.Cu") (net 2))
 (segment (start 50.0475 18.7775) (end 50.825 18) (width 0.2) (layer "F.Cu") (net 2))
 (segment (start 18.95 10) (end 18.95 11.6446) (width 0.2) (layer "F.Cu") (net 2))
 (segment (start 35.6025 18.7775) (end 42.0475 18.7775) (width 0.2) (layer "F.Cu") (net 2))
 (segment (start 86.75 5.1123) (end 85.9564 5.1123) (width 0.2) (layer "F.Cu") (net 2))
 (segment (start 18.825 18) (end 19.6025 18.7775) (width 0.2) (layer "F.Cu") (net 2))
 (segment (start 34.0475 18.7775) (end 27.6025 18.7775) (width 0.2) (layer "F.Cu") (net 2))
 (segment (start 26.0475 18.7775) (end 26.825 18) (width 0.2) (layer "F.Cu") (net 2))
 (segment (start 51.9763 19.1513) (end 68.1946 19.1513) (width 0.2) (layer "F.Cu") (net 2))
 (segment (start 81.3867 5.9592) (end 81.3888 5.9592) (width 0.2) (layer "F.Cu") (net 2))
 (segment (start 18.825 15.1549) (end 18.825 18) (width 0.2) (layer "F.Cu") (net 2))
 (segment (start 18.95 13.1319) (end 17.876 14.2059) (width 0.2) (layer "F.Cu") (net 2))
 (segment (start 81.3888 5.9592) (end 82.2269 5.1211) (width 0.2) (layer "F.Cu") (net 2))
 (segment (start 50.825 18) (end 51.9763 19.1513) (width 0.2) (layer "F.Cu") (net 2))
 (segment (start 17.876 14.2059) (end 18.825 15.1549) (width 0.2) (layer "F.Cu") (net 2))
 (segment (start 42.825 18) (end 43.6025 18.7775) (width 0.2) (layer "F.Cu") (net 2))
 (segment (start 10.825 18) (end 11.8122 17.0128) (width 0.2) (layer "F.Cu") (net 2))
 (segment (start 27.6025 18.7775) (end 26.825 18) (width 0.2) (layer "F.Cu") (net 2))
 (segment (start 11.8122 14.2059) (end 17.876 14.2059) (width 0.2) (layer "F.Cu") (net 2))
 (segment (start 93.25 5.955) (end 93.25 4.8476) (width 0.2) (layer "F.Cu") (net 2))
 (segment (start 42.0475 18.7775) (end 42.825 18) (width 0.2) (layer "F.Cu") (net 2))
 (segment (start 34.825 18) (end 34.0475 18.7775) (width 0.2) (layer "F.Cu") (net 2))
 (segment (start 11.8122 17.0128) (end 11.8122 14.2059) (width 0.2) (layer "F.Cu") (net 2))
 (segment (start 43.6025 18.7775) (end 50.0475 18.7775) (width 0.2) (layer "F.Cu") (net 2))
 (segment (start 34.825 18) (end 35.6025 18.7775) (width 0.2) (layer "F.Cu") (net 2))
 (segment (start 85.9564 5.1123) (end 85.9476 5.1211) (width 0.2) (layer "F.Cu") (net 2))
 (segment (start 18.95 11.6446) (end 18.95 13.1319) (width 0.2) (layer "F.Cu") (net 2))
 (segment (start 86.75 5.955) (end 86.75 5.1123) (width 0.2) (layer "F.Cu") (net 2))
 (segment (start 11.8122 14.2059) (end 11.8122 11.0372) (width 0.2) (layer "F.Cu") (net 2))
 (segment (start 68.1946 19.1513) (end 81.3867 5.9592) (width 0.2) (layer "F.Cu") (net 2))
 (segment (start 28 10) (end 26.3554 11.6446) (width 0.2) (layer "F.Cu") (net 2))
 (segment (start 82.2269 5.1211) (end 85.9476 5.1211) (width 0.2) (layer "F.Cu") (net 2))
 (segment (start 19.6025 18.7775) (end 26.0475 18.7775) (width 0.2) (layer "F.Cu") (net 2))
 (via (at 85.9476 5.1211) (size 0.6) (drill 0.3) (layers "F.Cu" "B.Cu") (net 2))
 (via (at 93.121 4.7186) (size 0.6) (drill 0.3) (layers "F.Cu" "B.Cu") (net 2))
 (segment (start 92.7185 5.1211) (end 93.121 4.7186) (width 0.2) (layer "B.Cu") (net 2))
 (segment (start 85.9476 5.1211) (end 92.7185 5.1211) (width 0.2) (layer "B.Cu") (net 2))
 (segment (start 33.2125 10) (end 33.175 10) (width 0.2) (layer "F.Cu") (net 16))
 (segment (start 33.175 10) (end 25.175 18) (width 0.2) (layer "F.Cu") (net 16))
 (segment (start 41.2125 10) (end 33.2125 18) (width 0.2) (layer "F.Cu") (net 4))
 (segment (start 33.2125 18) (end 33.175 18) (width 0.2) (layer "F.Cu") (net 4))
 (segment (start 49.2125 10) (end 41.2125 18) (width 0.2) (layer "F.Cu") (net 15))
 (segment (start 41.2125 18) (end 41.175 18) (width 0.2) (layer "F.Cu") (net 15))
 (segment (start 49.2125 18) (end 49.175 18) (width 0.2) (layer "F.Cu") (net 1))
 (segment (start 57.2125 10) (end 49.2125 18) (width 0.2) (layer "F.Cu") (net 1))
 (segment (start 62.9259 8.3259) (end 64.6 10) (width 0.2) (layer "F.Cu") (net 5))
 (segment (start 25.6741 8.3259) (end 62.9259 8.3259) (width 0.2) (layer "F.Cu") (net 5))
 (segment (start 87.55 5.0291) (end 87.0399 4.519) (width 0.2) (layer "F.Cu") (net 5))
 (segment (start 24 10) (end 25.6741 8.3259) (width 0.2) (layer "F.Cu") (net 5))
 (segment (start 87.0399 4.519) (end 70.081 4.519) (width 0.2) (layer "F.Cu") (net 5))
 (segment (start 92.45 4.9283) (end 87.6508 4.9283) (width 0.2) (layer "F.Cu") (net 5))
 (segment (start 87.6508 4.9283) (end 87.55 5.0291) (width 0.2) (layer "F.Cu") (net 5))
 (segment (start 70.081 4.519) (end 64.6 10) (width 0.2) (layer "F.Cu") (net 5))
 (segment (start 92.45 5.955) (end 92.45 4.9283) (width 0.2) (layer "F.Cu") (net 5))
 (segment (start 87.55 5.955) (end 87.55 5.0291) (width 0.2) (layer "F.Cu") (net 5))
 (segment (start 54.906 18.716) (end 54.19 18) (width 0.2) (layer "F.Cu") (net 14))
 (segment (start 67.4 10) (end 67.4 13.9451) (width 0.2) (layer "F.Cu") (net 14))
 (segment (start 62.6291 18.716) (end 54.906 18.716) (width 0.2) (layer "F.Cu") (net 14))
 (segment (start 67.4 13.9451) (end 62.6291 18.716) (width 0.2) (layer "F.Cu") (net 14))
 (segment (start 49.9728 9.1853) (end 43.6022 9.1853) (width 0.2) (layer "F.Cu") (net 3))
 (segment (start 58.7875 10) (end 61.81 13.0225) (width 0.2) (layer "F.Cu") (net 3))
 (segment (start 26.7276 8.7684) (end 33.5559 8.7684) (width 0.2) (layer "F.Cu") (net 3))
 (segment (start 19.7907 8.9489) (end 22.0655 11.2237) (width 0.2) (layer "F.Cu") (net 3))
 (segment (start 43.6022 9.1853) (end 42.7875 10) (width 0.2) (layer "F.Cu") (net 3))
 (segment (start 9.225 10) (end 10.0222 9.2028) (width 0.2) (layer "F.Cu") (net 3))
 (segment (start 26 10.4316) (end 26 9.496) (width 0.2) (layer "F.Cu") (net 3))
 (segment (start 61.81 13.0225) (end 61.81 18) (width 0.2) (layer "F.Cu") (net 3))
 (segment (start 51.6065 9.181) (end 57.9685 9.181) (width 0.2) (layer "F.Cu") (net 3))
 (segment (start 10.0222 9.2028) (end 16.2528 9.2028) (width 0.2) (layer "F.Cu") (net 3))
 (segment (start 42.7875 10) (end 41.973 9.1855) (width 0.2) (layer "F.Cu") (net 3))
 (segment (start 33.5559 8.7684) (end 34.7875 10) (width 0.2) (layer "F.Cu") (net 3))
 (segment (start 22.0655 11.2237) (end 25.2079 11.2237) (width 0.2) (layer "F.Cu") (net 3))
 (segment (start 16.2528 9.2028) (end 17.05 10) (width 0.2) (layer "F.Cu") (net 3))
 (segment (start 41.973 9.1855) (end 35.602 9.1855) (width 0.2) (layer "F.Cu") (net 3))
 (segment (start 25.2079 11.2237) (end 26 10.4316) (width 0.2) (layer "F.Cu") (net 3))
 (segment (start 35.602 9.1855) (end 34.7875 10) (width 0.2) (layer "F.Cu") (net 3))
 (segment (start 26 9.496) (end 26.7276 8.7684) (width 0.2) (layer "F.Cu") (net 3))
 (segment (start 50.7875 10) (end 49.9728 9.1853) (width 0.2) (layer "F.Cu") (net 3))
 (segment (start 18.1011 8.9489) (end 19.7907 8.9489) (width 0.2) (layer "F.Cu") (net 3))
 (segment (start 57.9685 9.181) (end 58.7875 10) (width 0.2) (layer "F.Cu") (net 3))
 (segment (start 17.05 10) (end 18.1011 8.9489) (width 0.2) (layer "F.Cu") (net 3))
 (segment (start 50.7875 10) (end 51.6065 9.181) (width 0.2) (layer "F.Cu") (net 3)))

